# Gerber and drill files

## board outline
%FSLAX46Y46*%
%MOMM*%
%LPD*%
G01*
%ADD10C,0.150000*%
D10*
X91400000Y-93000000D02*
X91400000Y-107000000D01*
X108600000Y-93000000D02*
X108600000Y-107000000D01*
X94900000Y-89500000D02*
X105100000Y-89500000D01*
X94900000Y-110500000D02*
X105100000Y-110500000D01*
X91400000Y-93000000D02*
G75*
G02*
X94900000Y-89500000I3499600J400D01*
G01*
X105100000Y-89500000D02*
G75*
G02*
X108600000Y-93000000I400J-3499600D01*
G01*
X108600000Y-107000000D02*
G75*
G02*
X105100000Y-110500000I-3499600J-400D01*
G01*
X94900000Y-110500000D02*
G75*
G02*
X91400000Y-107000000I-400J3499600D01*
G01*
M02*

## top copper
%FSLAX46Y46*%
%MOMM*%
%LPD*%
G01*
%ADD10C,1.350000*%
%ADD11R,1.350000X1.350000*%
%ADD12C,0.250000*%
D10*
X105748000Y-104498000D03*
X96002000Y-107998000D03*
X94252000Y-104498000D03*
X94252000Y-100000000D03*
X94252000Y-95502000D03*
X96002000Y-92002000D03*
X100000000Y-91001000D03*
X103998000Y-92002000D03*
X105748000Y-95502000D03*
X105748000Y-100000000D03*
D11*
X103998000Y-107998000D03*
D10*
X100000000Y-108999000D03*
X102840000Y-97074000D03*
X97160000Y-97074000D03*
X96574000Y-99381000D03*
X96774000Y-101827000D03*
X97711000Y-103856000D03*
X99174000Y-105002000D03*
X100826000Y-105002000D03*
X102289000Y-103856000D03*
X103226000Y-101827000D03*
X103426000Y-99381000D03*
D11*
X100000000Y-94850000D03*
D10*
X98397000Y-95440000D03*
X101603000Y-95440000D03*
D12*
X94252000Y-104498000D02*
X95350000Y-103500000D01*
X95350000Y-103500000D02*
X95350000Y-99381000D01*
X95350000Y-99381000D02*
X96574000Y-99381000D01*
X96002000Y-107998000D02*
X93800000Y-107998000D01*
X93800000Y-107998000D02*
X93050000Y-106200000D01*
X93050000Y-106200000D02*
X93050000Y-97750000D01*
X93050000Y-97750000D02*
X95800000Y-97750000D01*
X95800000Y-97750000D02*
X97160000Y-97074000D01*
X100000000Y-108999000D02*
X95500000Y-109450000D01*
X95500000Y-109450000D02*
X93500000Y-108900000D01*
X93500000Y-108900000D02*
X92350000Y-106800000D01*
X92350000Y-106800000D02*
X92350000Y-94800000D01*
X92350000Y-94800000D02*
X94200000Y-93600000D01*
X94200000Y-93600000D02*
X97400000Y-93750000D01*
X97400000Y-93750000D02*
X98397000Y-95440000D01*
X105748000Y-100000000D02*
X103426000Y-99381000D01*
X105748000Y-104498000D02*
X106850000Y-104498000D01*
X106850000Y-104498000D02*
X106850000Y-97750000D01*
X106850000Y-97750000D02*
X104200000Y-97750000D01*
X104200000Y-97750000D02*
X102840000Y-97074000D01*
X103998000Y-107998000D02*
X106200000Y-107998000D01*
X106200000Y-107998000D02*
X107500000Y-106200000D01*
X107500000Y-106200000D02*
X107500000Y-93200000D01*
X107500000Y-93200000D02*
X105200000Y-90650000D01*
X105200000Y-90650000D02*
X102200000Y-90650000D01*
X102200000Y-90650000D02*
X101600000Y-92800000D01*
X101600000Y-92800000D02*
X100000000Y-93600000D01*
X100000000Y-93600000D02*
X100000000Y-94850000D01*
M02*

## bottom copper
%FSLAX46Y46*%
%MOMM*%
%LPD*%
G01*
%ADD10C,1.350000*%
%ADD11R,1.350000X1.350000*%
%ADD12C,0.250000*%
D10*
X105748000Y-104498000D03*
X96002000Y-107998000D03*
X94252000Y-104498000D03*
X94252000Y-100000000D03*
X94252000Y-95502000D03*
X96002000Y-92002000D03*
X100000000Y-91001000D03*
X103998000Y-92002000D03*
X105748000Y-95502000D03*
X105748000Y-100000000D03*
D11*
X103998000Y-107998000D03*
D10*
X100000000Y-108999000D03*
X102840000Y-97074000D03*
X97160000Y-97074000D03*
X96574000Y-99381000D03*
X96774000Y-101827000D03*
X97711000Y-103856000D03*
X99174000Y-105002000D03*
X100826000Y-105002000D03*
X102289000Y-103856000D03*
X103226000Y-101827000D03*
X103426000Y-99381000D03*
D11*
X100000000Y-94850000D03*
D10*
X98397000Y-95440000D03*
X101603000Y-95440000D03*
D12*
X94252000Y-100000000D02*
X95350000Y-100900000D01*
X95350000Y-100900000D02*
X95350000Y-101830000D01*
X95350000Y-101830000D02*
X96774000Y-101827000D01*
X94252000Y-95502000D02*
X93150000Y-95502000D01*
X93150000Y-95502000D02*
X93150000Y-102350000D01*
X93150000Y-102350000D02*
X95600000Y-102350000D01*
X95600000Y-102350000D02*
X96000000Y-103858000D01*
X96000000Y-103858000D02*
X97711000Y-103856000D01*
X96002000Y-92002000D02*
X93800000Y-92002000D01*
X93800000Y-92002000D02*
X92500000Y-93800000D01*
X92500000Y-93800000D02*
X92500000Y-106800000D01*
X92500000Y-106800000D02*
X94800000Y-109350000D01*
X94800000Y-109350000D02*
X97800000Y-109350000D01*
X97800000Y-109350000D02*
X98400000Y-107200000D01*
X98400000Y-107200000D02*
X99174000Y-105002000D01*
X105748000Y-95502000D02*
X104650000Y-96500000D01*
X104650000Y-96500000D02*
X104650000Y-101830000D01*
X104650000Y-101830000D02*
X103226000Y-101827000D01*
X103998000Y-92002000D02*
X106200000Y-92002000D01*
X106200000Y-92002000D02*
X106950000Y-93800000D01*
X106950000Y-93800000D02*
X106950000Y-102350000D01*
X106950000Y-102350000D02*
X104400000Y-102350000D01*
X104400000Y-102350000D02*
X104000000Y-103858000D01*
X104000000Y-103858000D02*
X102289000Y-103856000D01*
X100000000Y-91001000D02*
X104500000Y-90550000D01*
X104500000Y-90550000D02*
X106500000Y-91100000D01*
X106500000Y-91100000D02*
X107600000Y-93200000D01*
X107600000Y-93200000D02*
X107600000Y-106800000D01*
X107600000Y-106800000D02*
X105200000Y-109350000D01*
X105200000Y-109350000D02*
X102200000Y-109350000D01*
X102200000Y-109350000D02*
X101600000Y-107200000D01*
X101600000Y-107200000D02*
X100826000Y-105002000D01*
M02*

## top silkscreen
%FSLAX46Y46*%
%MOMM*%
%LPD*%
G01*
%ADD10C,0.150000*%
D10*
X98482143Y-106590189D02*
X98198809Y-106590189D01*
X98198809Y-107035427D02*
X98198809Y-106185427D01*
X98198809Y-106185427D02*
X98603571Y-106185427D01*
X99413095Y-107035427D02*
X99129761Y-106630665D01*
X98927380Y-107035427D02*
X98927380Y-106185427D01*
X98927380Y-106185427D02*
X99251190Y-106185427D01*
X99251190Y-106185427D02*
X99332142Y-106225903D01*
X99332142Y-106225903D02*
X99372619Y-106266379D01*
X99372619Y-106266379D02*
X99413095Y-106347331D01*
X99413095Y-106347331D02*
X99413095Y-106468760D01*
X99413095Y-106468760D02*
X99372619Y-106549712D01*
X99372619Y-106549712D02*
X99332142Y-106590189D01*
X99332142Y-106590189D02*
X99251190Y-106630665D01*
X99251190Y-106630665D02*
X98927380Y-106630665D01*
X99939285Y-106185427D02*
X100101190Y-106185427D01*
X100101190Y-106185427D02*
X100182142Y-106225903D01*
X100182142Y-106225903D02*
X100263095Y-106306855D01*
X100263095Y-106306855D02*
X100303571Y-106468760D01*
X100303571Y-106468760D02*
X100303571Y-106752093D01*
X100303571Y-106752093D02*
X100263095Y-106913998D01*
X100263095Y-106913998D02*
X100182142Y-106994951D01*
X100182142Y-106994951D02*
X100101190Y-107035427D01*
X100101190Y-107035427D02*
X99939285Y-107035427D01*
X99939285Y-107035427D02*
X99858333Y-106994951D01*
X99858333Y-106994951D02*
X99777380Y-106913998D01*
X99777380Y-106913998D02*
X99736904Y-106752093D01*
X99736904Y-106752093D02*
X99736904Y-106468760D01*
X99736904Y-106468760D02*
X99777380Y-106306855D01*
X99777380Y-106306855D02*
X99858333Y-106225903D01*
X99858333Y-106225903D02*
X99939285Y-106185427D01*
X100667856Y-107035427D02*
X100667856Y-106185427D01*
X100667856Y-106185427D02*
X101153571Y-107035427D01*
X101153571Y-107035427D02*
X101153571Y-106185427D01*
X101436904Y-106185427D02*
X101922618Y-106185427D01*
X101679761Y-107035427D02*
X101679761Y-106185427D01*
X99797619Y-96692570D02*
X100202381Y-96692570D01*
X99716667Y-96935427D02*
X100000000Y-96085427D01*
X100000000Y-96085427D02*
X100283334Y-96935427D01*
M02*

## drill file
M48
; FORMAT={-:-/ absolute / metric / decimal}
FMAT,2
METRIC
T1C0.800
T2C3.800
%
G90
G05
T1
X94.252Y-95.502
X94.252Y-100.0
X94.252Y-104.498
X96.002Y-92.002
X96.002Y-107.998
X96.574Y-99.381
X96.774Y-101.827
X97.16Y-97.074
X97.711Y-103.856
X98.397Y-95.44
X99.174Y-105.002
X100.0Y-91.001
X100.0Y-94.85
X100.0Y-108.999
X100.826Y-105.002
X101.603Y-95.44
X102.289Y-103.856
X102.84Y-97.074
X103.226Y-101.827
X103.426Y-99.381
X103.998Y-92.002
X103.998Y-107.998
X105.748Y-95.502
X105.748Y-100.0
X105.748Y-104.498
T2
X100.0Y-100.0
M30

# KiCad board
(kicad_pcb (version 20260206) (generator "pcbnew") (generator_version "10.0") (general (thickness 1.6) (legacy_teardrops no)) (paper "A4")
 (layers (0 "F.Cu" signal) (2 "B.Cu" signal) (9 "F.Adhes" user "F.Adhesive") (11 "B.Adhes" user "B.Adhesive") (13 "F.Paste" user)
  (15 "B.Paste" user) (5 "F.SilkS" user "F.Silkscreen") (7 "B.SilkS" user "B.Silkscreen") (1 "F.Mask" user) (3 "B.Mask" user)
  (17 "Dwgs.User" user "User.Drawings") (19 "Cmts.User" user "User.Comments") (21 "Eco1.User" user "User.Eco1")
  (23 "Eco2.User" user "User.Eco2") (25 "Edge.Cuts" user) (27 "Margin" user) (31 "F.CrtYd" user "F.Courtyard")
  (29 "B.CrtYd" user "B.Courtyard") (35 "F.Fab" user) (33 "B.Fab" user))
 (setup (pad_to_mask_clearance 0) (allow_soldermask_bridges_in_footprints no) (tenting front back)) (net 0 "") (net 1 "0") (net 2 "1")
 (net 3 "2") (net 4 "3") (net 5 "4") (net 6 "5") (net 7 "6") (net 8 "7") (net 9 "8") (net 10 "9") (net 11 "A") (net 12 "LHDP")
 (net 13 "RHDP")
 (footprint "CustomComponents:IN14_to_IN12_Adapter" (layer "F.Cu") (at 100.000 100.000)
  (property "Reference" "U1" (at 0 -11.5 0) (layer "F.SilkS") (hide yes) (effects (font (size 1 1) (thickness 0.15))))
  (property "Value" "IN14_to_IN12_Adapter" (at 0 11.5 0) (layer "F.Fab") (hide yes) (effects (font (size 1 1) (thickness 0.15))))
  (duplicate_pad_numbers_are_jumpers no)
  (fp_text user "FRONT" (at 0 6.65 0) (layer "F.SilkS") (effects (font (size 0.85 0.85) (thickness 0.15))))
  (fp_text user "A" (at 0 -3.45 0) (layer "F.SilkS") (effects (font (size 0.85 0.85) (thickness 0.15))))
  (pad "" np_thru_hole circle (at 0 0) (size 3.8 3.8) (drill 3.8) (layers "*.Cu" "*.Mask"))
  (pad "0" thru_hole circle (at 5.748 4.498) (size 1.35 1.35) (drill 0.8) (layers "*.Cu" "*.Mask") (remove_unused_layers no) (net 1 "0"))
  (pad "1" thru_hole circle (at -3.998 7.998) (size 1.35 1.35) (drill 0.8) (layers "*.Cu" "*.Mask") (remove_unused_layers no) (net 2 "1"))
  (pad "2" thru_hole circle (at -5.748 4.498) (size 1.35 1.35) (drill 0.8) (layers "*.Cu" "*.Mask") (remove_unused_layers no) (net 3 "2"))
  (pad "3" thru_hole circle (at -5.748 0.000) (size 1.35 1.35) (drill 0.8) (layers "*.Cu" "*.Mask") (remove_unused_layers no) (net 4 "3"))
  (pad "4" thru_hole circle (at -5.748 -4.498) (size 1.35 1.35) (drill 0.8) (layers "*.Cu" "*.Mask") (remove_unused_layers no) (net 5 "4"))
  (pad "5" thru_hole circle (at -3.998 -7.998) (size 1.35 1.35) (drill 0.8) (layers "*.Cu" "*.Mask") (remove_unused_layers no) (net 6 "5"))
  (pad "6" thru_hole circle (at 0.000 -8.999) (size 1.35 1.35) (drill 0.8) (layers "*.Cu" "*.Mask") (remove_unused_layers no) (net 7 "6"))
  (pad "7" thru_hole circle (at 3.998 -7.998) (size 1.35 1.35) (drill 0.8) (layers "*.Cu" "*.Mask") (remove_unused_layers no) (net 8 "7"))
  (pad "8" thru_hole circle (at 5.748 -4.498) (size 1.35 1.35) (drill 0.8) (layers "*.Cu" "*.Mask") (remove_unused_layers no) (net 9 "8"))
  (pad "9" thru_hole circle (at 5.748 0.000) (size 1.35 1.35) (drill 0.8) (layers "*.Cu" "*.Mask") (remove_unused_layers no) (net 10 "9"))
  (pad "A" thru_hole rect (at 3.998 7.998) (size 1.35 1.35) (drill 0.8) (layers "*.Cu" "*.Mask") (remove_unused_layers no) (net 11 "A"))
  (pad "LHDP" thru_hole circle (at 0.000 8.999) (size 1.35 1.35) (drill 0.8) (layers "*.Cu" "*.Mask") (remove_unused_layers no)
   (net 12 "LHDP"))
  (pad "0" thru_hole circle (at 2.840 -2.926) (size 1.35 1.35) (drill 0.8) (layers "*.Cu" "*.Mask") (remove_unused_layers no) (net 1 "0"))
  (pad "1" thru_hole circle (at -2.840 -2.926) (size 1.35 1.35) (drill 0.8) (layers "*.Cu" "*.Mask") (remove_unused_layers no) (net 2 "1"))
  (pad "2" thru_hole circle (at -3.426 -0.619) (size 1.35 1.35) (drill 0.8) (layers "*.Cu" "*.Mask") (remove_unused_layers no) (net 3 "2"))
  (pad "3" thru_hole circle (at -3.226 1.827) (size 1.35 1.35) (drill 0.8) (layers "*.Cu" "*.Mask") (remove_unused_layers no) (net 4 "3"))
  (pad "4" thru_hole circle (at -2.289 3.856) (size 1.35 1.35) (drill 0.8) (layers "*.Cu" "*.Mask") (remove_unused_layers no) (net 5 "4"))
  (pad "5" thru_hole circle (at -0.826 5.002) (size 1.35 1.35) (drill 0.8) (layers "*.Cu" "*.Mask") (remove_unused_layers no) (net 6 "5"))
  (pad "6" thru_hole circle (at 0.826 5.002) (size 1.35 1.35) (drill 0.8) (layers "*.Cu" "*.Mask") (remove_unused_layers no) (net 7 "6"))
  (pad "7" thru_hole circle (at 2.289 3.856) (size 1.35 1.35) (drill 0.8) (layers "*.Cu" "*.Mask") (remove_unused_layers no) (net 8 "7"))
  (pad "8" thru_hole circle (at 3.226 1.827) (size 1.35 1.35) (drill 0.8) (layers "*.Cu" "*.Mask") (remove_unused_layers no) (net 9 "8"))
  (pad "9" thru_hole circle (at 3.426 -0.619) (size 1.35 1.35) (drill 0.8) (layers "*.Cu" "*.Mask") (remove_unused_layers no) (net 10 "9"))
  (pad "A" thru_hole rect (at -0.000 -5.150) (size 1.35 1.35) (drill 0.8) (layers "*.Cu" "*.Mask") (remove_unused_layers no) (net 11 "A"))
  (pad "LHDP" thru_hole circle (at -1.603 -4.560) (size 1.35 1.35) (drill 0.8) (layers "*.Cu" "*.Mask") (remove_unused_layers no)
   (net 12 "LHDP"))
  (pad "RHDP" thru_hole circle (at 1.603 -4.560) (size 1.35 1.35) (drill 0.8) (layers "*.Cu" "*.Mask") (remove_unused_layers no)
   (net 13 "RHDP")))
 (gr_line (start 91.400 93.000) (end 91.400 107.000) (stroke (width 0.15) (type solid)) (layer "Edge.Cuts"))
 (gr_line (start 108.600 93.000) (end 108.600 107.000) (stroke (width 0.15) (type solid)) (layer "Edge.Cuts"))
 (gr_line (start 94.900 89.500) (end 105.100 89.500) (stroke (width 0.15) (type solid)) (layer "Edge.Cuts"))
 (gr_line (start 94.900 110.500) (end 105.100 110.500) (stroke (width 0.15) (type solid)) (layer "Edge.Cuts"))
 (gr_arc (start 91.400 93.000) (mid 92.425 90.525) (end 94.900 89.500) (stroke (width 0.15) (type solid)) (layer "Edge.Cuts"))
 (gr_arc (start 105.100 89.500) (mid 107.575 90.525) (end 108.600 93.000) (stroke (width 0.15) (type solid)) (layer "Edge.Cuts"))
 (gr_arc (start 108.600 107.000) (mid 107.575 109.475) (end 105.100 110.500) (stroke (width 0.15) (type solid)) (layer "Edge.Cuts"))
 (gr_arc (start 94.900 110.500) (mid 92.425 109.475) (end 91.400 107.000) (stroke (width 0.15) (type solid)) (layer "Edge.Cuts"))
 (segment (start 94.252 104.498) (end 95.350 103.500) (width 0.25) (layer "F.Cu") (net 3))
 (segment (start 95.350 103.500) (end 95.350 99.381) (width 0.25) (layer "F.Cu") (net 3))
 (segment (start 95.350 99.381) (end 96.574 99.381) (width 0.25) (layer "F.Cu") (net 3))
 (segment (start 96.002 107.998) (end 93.800 107.998) (width 0.25) (layer "F.Cu") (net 2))
 (segment (start 93.800 107.998) (end 93.050 106.200) (width 0.25) (layer "F.Cu") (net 2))
 (segment (start 93.050 106.200) (end 93.050 97.750) (width 0.25) (layer "F.Cu") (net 2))
 (segment (start 93.050 97.750) (end 95.800 97.750) (width 0.25) (layer "F.Cu") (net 2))
 (segment (start 95.800 97.750) (end 97.160 97.074) (width 0.25) (layer "F.Cu") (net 2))
 (segment (start 100.000 108.999) (end 95.500 109.450) (width 0.25) (layer "F.Cu") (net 12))
 (segment (start 95.500 109.450) (end 93.500 108.900) (width 0.25) (layer "F.Cu") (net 12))
 (segment (start 93.500 108.900) (end 92.350 106.800) (width 0.25) (layer "F.Cu") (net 12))
 (segment (start 92.350 106.800) (end 92.350 94.800) (width 0.25) (layer "F.Cu") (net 12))
 (segment (start 92.350 94.800) (end 94.200 93.600) (width 0.25) (layer "F.Cu") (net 12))
 (segment (start 94.200 93.600) (end 97.400 93.750) (width 0.25) (layer "F.Cu") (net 12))
 (segment (start 97.400 93.750) (end 98.397 95.440) (width 0.25) (layer "F.Cu") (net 12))
 (segment (start 105.748 100.000) (end 103.426 99.381) (width 0.25) (layer "F.Cu") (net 10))
 (segment (start 105.748 104.498) (end 106.850 104.498) (width 0.25) (layer "F.Cu") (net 1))
 (segment (start 106.850 104.498) (end 106.850 97.750) (width 0.25) (layer "F.Cu") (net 1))
 (segment (start 106.850 97.750) (end 104.200 97.750) (width 0.25) (layer "F.Cu") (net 1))
 (segment (start 104.200 97.750) (end 102.840 97.074) (width 0.25) (layer "F.Cu") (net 1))
 (segment (start 103.998 107.998) (end 106.200 107.998) (width 0.25) (layer "F.Cu") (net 11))
 (segment (start 106.200 107.998) (end 107.500 106.200) (width 0.25) (layer "F.Cu") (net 11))
 (segment (start 107.500 106.200) (end 107.500 93.200) (width 0.25) (layer "F.Cu") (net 11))
 (segment (start 107.500 93.200) (end 105.200 90.650) (width 0.25) (layer "F.Cu") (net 11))
 (segment (start 105.200 90.650) (end 102.200 90.650) (width 0.25) (layer "F.Cu") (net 11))
 (segment (start 102.200 90.650) (end 101.600 92.800) (width 0.25) (layer "F.Cu") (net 11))
 (segment (start 101.600 92.800) (end 100.000 93.600) (width 0.25) (layer "F.Cu") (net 11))
 (segment (start 100.000 93.600) (end 100.000 94.850) (width 0.25) (layer "F.Cu") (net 11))
 (segment (start 94.252 100.000) (end 95.350 100.900) (width 0.25) (layer "B.Cu") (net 4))
 (segment (start 95.350 100.900) (end 95.350 101.830) (width 0.25) (layer "B.Cu") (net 4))
 (segment (start 95.350 101.830) (end 96.774 101.827) (width 0.25) (layer "B.Cu") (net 4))
 (segment (start 94.252 95.502) (end 93.150 95.502) (width 0.25) (layer "B.Cu") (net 5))
 (segment (start 93.150 95.502) (end 93.150 102.350) (width 0.25) (layer "B.Cu") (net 5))
 (segment (start 93.150 102.350) (end 95.600 102.350) (width 0.25) (layer "B.Cu") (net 5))
 (segment (start 95.600 102.350) (end 96.000 103.858) (width 0.25) (layer "B.Cu") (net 5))
 (segment (start 96.000 103.858) (end 97.711 103.856) (width 0.25) (layer "B.Cu") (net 5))
 (segment (start 96.002 92.002) (end 93.800 92.002) (width 0.25) (layer "B.Cu") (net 6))
 (segment (start 93.800 92.002) (end 92.500 93.800) (width 0.25) (layer "B.Cu") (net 6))
 (segment (start 92.500 93.800) (end 92.500 106.800) (width 0.25) (layer "B.Cu") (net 6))
 (segment (start 92.500 106.800) (end 94.800 109.350) (width 0.25) (layer "B.Cu") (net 6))
 (segment (start 94.800 109.350) (end 97.800 109.350) (width 0.25) (layer "B.Cu") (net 6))
 (segment (start 97.800 109.350) (end 98.400 107.200) (width 0.25) (layer "B.Cu") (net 6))
 (segment (start 98.400 107.200) (end 99.174 105.002) (width 0.25) (layer "B.Cu") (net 6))
 (segment (start 105.748 95.502) (end 104.650 96.500) (width 0.25) (layer "B.Cu") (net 9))
 (segment (start 104.650 96.500) (end 104.650 101.830) (width 0.25) (layer "B.Cu") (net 9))
 (segment (start 104.650 101.830) (end 103.226 101.827) (width 0.25) (layer "B.Cu") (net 9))
 (segment (start 103.998 92.002) (end 106.200 92.002) (width 0.25) (layer "B.Cu") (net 8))
 (segment (start 106.200 92.002) (end 106.950 93.800) (width 0.25) (layer "B.Cu") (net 8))
 (segment (start 106.950 93.800) (end 106.950 102.350) (width 0.25) (layer "B.Cu") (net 8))
 (segment (start 106.950 102.350) (end 104.400 102.350) (width 0.25) (layer "B.Cu") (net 8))
 (segment (start 104.400 102.350) (end 104.000 103.858) (width 0.25) (layer "B.Cu") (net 8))
 (segment (start 104.000 103.858) (end 102.289 103.856) (width 0.25) (layer "B.Cu") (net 8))
 (segment (start 100.000 91.001) (end 104.500 90.550) (width 0.25) (layer "B.Cu") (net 7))
 (segment (start 104.500 90.550) (end 106.500 91.100) (width 0.25) (layer "B.Cu") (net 7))
 (segment (start 106.500 91.100) (end 107.600 93.200) (width 0.25) (layer "B.Cu") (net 7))
 (segment (start 107.600 93.200) (end 107.600 106.800) (width 0.25) (layer "B.Cu") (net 7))
 (segment (start 107.600 106.800) (end 105.200 109.350) (width 0.25) (layer "B.Cu") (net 7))
 (segment (start 105.200 109.350) (end 102.200 109.350) (width 0.25) (layer "B.Cu") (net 7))
 (segment (start 102.200 109.350) (end 101.600 107.200) (width 0.25) (layer "B.Cu") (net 7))
 (segment (start 101.600 107.200) (end 100.826 105.002) (width 0.25) (layer "B.Cu") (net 7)))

